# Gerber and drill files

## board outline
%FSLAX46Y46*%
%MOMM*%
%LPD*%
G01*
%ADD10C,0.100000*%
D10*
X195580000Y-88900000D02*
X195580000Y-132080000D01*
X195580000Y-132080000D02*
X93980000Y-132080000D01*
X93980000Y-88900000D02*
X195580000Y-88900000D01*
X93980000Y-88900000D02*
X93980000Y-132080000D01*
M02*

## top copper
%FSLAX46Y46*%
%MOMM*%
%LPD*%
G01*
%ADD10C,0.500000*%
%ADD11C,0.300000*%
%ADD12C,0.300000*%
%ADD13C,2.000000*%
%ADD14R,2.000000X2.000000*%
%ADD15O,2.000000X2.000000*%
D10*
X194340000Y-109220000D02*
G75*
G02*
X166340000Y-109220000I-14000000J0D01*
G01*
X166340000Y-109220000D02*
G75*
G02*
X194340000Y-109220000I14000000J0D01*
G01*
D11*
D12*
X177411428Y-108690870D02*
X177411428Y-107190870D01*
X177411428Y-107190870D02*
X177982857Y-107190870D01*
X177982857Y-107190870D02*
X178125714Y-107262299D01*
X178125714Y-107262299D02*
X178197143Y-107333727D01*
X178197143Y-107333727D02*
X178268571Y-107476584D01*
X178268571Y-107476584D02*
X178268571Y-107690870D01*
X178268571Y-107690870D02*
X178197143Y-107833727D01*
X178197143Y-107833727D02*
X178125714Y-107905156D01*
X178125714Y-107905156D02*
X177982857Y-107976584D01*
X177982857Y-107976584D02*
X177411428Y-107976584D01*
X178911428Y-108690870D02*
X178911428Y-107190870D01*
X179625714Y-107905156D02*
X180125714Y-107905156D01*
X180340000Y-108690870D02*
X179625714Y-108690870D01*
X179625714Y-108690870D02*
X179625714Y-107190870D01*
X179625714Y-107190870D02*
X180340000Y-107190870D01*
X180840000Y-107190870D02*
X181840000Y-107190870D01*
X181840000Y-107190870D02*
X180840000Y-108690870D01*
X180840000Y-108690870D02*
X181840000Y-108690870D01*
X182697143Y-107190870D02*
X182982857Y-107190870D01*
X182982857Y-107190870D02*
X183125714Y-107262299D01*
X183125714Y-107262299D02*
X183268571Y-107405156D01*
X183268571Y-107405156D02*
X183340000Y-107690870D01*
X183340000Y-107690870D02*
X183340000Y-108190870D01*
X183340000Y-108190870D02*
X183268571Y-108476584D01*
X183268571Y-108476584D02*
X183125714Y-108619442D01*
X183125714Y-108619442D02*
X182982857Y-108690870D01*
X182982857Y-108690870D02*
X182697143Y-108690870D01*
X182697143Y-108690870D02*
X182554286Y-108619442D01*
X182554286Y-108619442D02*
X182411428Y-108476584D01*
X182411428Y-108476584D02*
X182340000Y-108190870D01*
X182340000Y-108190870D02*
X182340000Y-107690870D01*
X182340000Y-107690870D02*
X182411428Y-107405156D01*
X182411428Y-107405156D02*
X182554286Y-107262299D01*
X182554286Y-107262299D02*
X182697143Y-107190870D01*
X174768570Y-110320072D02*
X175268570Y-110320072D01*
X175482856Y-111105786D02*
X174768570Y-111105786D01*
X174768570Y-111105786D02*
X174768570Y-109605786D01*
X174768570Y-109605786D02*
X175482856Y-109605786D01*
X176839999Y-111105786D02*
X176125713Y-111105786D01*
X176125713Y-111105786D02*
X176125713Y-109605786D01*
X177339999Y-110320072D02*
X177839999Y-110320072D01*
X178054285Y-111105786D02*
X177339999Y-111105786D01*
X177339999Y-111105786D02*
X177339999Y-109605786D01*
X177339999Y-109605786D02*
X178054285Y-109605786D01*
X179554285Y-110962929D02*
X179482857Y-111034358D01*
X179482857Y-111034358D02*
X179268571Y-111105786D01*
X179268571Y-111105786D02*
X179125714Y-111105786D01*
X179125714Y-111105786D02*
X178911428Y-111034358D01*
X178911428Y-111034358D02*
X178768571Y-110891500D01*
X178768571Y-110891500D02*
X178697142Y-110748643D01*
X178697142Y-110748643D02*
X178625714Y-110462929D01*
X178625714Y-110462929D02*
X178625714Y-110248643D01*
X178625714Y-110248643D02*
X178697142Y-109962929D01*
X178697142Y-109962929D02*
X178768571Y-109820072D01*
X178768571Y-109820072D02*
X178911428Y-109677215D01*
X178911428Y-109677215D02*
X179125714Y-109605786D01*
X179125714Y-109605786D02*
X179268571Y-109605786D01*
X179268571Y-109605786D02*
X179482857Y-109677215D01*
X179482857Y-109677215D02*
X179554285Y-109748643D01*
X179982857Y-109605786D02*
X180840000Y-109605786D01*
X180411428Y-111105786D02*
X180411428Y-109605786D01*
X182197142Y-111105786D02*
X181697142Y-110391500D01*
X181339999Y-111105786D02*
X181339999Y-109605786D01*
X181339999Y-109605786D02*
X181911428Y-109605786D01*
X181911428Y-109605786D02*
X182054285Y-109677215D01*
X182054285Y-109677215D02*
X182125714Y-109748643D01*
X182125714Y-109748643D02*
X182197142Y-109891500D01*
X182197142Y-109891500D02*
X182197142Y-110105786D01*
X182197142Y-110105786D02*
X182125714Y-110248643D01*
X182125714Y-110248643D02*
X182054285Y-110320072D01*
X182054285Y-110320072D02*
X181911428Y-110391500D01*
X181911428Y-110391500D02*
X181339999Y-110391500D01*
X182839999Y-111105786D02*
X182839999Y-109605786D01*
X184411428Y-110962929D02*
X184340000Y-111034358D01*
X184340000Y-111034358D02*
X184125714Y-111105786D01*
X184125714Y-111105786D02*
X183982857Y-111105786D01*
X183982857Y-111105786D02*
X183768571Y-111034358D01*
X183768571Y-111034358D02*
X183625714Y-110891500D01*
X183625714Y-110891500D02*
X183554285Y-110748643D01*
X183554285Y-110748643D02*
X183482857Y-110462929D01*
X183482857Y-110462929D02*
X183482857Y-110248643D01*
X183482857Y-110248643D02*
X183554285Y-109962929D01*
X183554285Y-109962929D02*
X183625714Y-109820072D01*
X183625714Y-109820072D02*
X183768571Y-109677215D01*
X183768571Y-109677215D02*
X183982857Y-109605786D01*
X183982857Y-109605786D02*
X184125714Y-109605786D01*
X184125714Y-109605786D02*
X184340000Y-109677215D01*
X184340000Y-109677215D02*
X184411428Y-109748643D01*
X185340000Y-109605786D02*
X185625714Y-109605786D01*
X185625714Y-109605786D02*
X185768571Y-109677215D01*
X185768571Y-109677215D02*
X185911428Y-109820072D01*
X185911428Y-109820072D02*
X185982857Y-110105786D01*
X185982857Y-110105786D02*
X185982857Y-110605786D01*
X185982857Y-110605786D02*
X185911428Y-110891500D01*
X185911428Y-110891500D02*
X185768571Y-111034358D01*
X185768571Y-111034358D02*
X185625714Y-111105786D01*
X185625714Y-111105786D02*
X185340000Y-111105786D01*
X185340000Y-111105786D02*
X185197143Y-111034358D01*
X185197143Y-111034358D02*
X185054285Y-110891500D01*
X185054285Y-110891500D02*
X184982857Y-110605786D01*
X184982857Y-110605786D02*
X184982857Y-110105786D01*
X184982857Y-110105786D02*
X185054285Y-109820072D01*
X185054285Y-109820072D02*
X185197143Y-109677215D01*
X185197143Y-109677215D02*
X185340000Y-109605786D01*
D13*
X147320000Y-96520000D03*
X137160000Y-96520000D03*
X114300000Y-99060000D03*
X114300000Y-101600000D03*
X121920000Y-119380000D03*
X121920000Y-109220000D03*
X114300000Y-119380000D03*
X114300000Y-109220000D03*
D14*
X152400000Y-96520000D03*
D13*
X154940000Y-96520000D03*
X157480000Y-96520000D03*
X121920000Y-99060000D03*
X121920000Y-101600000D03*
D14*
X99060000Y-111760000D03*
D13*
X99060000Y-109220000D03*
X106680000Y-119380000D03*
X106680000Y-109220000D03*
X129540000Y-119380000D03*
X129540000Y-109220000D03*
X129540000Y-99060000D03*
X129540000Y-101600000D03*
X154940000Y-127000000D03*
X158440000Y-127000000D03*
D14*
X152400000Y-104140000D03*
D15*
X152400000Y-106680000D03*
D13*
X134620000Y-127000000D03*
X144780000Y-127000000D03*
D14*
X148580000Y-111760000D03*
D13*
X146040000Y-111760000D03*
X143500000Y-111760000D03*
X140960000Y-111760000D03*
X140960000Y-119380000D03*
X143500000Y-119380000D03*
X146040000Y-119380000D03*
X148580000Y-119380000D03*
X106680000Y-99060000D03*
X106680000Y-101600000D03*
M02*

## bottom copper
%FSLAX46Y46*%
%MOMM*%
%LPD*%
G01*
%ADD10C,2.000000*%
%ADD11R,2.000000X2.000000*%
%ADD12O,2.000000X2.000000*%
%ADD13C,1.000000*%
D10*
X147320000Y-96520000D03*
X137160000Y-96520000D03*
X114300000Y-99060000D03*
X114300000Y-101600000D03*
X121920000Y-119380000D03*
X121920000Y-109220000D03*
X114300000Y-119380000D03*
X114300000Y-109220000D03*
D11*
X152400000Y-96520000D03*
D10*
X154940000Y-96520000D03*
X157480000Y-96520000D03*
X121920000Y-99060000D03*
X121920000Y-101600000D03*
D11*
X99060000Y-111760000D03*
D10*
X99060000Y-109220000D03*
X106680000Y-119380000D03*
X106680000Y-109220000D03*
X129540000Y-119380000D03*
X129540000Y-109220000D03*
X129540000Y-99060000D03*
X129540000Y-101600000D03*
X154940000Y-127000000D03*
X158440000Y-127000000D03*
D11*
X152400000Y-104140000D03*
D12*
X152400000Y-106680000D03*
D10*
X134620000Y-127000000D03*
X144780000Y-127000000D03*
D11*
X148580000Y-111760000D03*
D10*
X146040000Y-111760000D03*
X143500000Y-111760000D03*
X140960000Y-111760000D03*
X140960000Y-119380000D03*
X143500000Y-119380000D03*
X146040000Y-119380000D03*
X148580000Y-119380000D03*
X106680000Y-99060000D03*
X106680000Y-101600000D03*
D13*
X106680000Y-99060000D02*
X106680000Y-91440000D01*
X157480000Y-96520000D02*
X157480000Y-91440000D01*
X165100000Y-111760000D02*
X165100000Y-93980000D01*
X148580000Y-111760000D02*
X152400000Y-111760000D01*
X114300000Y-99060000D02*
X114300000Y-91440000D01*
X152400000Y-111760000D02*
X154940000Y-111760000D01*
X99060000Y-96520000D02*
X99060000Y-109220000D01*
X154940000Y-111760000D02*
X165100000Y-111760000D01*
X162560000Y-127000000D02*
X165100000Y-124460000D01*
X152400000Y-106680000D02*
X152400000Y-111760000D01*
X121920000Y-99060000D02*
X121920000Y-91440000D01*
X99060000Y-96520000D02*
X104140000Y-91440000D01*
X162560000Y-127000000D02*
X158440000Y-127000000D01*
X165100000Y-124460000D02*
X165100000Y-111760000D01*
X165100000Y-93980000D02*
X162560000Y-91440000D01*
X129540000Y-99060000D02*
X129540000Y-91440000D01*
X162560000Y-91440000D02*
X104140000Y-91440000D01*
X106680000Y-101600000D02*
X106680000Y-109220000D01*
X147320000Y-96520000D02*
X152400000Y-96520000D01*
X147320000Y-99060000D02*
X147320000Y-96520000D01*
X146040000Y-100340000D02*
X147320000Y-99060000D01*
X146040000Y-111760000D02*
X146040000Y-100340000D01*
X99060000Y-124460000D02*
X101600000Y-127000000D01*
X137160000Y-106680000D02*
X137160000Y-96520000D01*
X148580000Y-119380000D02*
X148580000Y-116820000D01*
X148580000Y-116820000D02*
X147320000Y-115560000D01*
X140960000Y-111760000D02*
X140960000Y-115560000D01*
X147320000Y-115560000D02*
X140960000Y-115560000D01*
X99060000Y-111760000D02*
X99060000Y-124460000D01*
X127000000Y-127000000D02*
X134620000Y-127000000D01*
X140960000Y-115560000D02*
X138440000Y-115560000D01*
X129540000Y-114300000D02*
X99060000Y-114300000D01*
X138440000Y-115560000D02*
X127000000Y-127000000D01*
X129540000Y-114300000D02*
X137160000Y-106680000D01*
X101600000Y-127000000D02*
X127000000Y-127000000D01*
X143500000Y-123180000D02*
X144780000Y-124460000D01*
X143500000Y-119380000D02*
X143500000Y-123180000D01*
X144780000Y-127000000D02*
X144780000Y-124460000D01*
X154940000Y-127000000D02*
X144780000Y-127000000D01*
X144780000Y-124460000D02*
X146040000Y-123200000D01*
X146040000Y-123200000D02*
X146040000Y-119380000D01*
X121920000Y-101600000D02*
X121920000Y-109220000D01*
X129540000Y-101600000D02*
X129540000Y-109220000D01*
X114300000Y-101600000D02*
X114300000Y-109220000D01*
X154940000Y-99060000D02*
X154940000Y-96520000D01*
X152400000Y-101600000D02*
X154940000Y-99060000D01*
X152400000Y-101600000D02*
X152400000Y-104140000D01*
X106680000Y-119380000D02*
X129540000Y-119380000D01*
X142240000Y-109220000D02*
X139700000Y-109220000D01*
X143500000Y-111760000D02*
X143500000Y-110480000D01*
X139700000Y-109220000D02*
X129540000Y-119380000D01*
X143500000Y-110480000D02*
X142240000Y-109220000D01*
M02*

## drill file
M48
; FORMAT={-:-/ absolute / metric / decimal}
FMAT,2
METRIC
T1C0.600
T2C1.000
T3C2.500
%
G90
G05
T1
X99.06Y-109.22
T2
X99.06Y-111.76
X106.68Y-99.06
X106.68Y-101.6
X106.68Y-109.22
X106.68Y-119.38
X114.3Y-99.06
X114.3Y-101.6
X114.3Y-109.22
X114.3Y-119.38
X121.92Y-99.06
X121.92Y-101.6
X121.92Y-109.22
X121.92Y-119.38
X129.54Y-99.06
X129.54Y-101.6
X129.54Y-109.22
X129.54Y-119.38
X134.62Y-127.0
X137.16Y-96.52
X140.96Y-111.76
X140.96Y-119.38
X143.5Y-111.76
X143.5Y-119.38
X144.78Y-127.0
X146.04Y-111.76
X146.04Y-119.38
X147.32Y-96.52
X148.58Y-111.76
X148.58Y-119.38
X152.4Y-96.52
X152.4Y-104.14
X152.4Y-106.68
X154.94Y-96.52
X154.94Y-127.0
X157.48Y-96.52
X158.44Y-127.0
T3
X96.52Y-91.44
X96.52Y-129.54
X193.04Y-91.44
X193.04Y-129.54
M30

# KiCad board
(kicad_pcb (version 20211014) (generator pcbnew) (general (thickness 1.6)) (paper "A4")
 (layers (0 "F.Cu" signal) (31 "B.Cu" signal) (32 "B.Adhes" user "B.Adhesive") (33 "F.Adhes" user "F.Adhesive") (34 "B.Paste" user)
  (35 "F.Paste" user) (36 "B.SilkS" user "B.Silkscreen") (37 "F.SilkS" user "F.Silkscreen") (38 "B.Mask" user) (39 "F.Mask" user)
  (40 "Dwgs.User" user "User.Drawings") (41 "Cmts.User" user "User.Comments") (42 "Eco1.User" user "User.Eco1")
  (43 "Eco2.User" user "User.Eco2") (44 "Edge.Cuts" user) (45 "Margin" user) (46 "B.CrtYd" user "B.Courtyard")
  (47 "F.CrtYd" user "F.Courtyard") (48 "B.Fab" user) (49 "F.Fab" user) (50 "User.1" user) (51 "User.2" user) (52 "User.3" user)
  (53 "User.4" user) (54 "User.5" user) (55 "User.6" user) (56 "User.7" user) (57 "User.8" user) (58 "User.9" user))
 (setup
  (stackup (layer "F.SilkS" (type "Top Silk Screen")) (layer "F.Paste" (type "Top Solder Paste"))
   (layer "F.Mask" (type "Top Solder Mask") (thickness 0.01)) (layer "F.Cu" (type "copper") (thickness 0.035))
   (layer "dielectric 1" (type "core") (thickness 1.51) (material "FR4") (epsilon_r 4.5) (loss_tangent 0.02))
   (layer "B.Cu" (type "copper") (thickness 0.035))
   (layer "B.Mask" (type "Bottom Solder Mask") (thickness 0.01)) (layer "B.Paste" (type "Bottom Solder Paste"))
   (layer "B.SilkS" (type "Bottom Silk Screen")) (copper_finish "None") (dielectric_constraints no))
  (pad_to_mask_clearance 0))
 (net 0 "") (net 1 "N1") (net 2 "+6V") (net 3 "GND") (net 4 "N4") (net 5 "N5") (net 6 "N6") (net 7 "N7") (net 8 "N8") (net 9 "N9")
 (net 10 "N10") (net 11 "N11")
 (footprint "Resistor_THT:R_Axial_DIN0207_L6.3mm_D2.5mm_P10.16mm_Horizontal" (layer "F.Cu") (at 147.32 96.52 180)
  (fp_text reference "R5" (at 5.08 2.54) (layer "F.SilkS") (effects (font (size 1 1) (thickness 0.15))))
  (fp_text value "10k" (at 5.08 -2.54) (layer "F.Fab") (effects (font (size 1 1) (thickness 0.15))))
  (pad "1" thru_hole circle (at 0 0 180) (size 2 2) (drill 1) (layers *.Cu *.Mask) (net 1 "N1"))
  (pad "2" thru_hole circle (at 10.16 0 180) (size 2 2) (drill 1) (layers *.Cu *.Mask) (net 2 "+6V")))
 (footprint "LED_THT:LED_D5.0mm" (layer "F.Cu") (at 114.3 99.06 -90)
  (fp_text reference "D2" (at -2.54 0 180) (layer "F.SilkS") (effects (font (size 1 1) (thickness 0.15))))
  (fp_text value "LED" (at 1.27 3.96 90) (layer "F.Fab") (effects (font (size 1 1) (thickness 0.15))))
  (pad "1" thru_hole circle (at 0 0 270) (size 2 2) (drill 1) (layers *.Cu *.Mask) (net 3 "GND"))
  (pad "2" thru_hole circle (at 2.54 0 270) (size 2 2) (drill 1) (layers *.Cu *.Mask) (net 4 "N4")))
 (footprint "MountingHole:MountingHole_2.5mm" (layer "F.Cu") (at 96.52 91.44)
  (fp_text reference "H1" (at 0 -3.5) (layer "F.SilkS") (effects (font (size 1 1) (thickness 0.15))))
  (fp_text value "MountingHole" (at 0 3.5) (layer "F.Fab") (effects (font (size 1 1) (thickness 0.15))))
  (pad "" np_thru_hole circle (at 0 0) (size 2.5 2.5) (drill 2.5) (layers *.Cu *.Mask)))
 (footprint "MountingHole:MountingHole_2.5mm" (layer "F.Cu") (at 96.52 129.54 180)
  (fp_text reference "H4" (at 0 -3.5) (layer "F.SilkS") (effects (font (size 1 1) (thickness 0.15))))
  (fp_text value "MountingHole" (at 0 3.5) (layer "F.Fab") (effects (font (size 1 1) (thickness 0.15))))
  (pad "" np_thru_hole circle (at 0 0 180) (size 2.5 2.5) (drill 2.5) (layers *.Cu *.Mask)))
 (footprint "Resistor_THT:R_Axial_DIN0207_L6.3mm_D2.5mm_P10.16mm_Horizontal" (layer "F.Cu") (at 121.92 119.38 90)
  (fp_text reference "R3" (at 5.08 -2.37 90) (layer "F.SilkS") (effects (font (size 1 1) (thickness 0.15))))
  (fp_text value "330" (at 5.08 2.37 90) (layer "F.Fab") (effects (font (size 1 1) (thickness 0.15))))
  (pad "1" thru_hole circle (at 0 0 90) (size 2 2) (drill 1) (layers *.Cu *.Mask) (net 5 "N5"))
  (pad "2" thru_hole circle (at 10.16 0 90) (size 2 2) (drill 1) (layers *.Cu *.Mask) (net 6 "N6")))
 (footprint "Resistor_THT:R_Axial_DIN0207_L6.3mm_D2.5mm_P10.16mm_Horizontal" (layer "F.Cu") (at 114.3 119.38 90)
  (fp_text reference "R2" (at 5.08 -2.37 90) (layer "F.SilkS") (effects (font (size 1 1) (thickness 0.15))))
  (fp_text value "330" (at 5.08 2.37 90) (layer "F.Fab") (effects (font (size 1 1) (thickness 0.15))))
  (pad "1" thru_hole circle (at 0 0 90) (size 2 2) (drill 1) (layers *.Cu *.Mask) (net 5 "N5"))
  (pad "2" thru_hole circle (at 10.16 0 90) (size 2 2) (drill 1) (layers *.Cu *.Mask) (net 4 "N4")))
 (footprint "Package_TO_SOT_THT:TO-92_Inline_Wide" (layer "F.Cu") (at 152.4 96.52)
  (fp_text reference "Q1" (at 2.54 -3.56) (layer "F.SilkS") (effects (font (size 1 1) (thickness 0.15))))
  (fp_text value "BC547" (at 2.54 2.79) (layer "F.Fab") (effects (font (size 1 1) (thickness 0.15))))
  (pad "1" thru_hole rect (at 0 0) (size 2 2) (drill 1) (layers *.Cu *.Mask) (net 1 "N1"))
  (pad "2" thru_hole circle (at 2.54 0) (size 2 2) (drill 1) (layers *.Cu *.Mask) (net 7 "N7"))
  (pad "3" thru_hole circle (at 5.08 0) (size 2 2) (drill 1) (layers *.Cu *.Mask) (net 3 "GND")))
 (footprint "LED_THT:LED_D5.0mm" (layer "F.Cu") (at 121.92 99.06 -90)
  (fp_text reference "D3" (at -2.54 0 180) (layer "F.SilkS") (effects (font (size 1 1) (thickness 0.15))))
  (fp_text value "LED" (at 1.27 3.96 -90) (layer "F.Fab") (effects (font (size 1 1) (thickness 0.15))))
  (pad "1" thru_hole circle (at 0 0 270) (size 2 2) (drill 1) (layers *.Cu *.Mask) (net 3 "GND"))
  (pad "2" thru_hole circle (at 2.54 0 270) (size 2 2) (drill 1) (layers *.Cu *.Mask) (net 6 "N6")))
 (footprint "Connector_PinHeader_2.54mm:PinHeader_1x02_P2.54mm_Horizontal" (layer "F.Cu") (at 99.06 111.76 180)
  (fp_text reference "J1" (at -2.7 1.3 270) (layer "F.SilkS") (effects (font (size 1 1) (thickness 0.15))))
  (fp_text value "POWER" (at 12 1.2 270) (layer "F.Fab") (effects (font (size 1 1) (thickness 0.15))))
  (pad "1" thru_hole rect (at 0 0 180) (size 2 2) (drill 1) (layers *.Cu *.Mask) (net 2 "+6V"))
  (pad "2" thru_hole circle (at 0 2.54 180) (size 2 2) (drill 0.6) (layers *.Cu *.Mask) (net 3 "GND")))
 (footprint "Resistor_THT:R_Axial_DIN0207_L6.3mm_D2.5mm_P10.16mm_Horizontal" (layer "F.Cu") (at 106.68 119.38 90)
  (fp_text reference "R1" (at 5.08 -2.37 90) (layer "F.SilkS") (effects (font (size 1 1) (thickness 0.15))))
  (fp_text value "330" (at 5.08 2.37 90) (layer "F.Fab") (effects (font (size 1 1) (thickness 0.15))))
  (pad "1" thru_hole circle (at 0 0 90) (size 2 2) (drill 1) (layers *.Cu *.Mask) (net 5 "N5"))
  (pad "2" thru_hole circle (at 10.16 0 90) (size 2 2) (drill 1) (layers *.Cu *.Mask) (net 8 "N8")))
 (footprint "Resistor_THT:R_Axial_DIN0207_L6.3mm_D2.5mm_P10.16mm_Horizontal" (layer "F.Cu") (at 129.54 119.38 90)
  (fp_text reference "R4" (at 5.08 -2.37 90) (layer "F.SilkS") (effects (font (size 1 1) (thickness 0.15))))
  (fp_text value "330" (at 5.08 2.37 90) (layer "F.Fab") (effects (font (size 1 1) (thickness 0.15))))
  (pad "1" thru_hole circle (at 0 0 90) (size 2 2) (drill 1) (layers *.Cu *.Mask) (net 5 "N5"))
  (pad "2" thru_hole circle (at 10.16 0 90) (size 2 2) (drill 1) (layers *.Cu *.Mask "Dwgs.User") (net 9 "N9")))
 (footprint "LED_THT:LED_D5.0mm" (layer "F.Cu") (at 129.54 99.06 -90)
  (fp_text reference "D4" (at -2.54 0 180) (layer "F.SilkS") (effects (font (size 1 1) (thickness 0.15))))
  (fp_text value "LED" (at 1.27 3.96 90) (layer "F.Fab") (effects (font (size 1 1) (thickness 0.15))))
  (pad "1" thru_hole circle (at 0 0 270) (size 2 2) (drill 1) (layers *.Cu *.Mask) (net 3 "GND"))
  (pad "2" thru_hole circle (at 2.54 0 270) (size 2 2) (drill 1) (layers *.Cu "B.Mask") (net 9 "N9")))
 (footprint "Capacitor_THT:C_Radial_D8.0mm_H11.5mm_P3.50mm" (layer "F.Cu") (at 154.94 127)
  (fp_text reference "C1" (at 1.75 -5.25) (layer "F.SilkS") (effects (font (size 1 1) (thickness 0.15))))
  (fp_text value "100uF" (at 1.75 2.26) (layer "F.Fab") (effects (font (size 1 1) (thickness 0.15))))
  (pad "1" thru_hole circle (at 0 0) (size 2 2) (drill 1) (layers *.Cu *.Mask) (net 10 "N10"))
  (pad "2" thru_hole circle (at 3.5 0) (size 2 2) (drill 1) (layers *.Cu *.Mask) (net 3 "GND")))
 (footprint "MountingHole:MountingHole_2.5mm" (layer "F.Cu") (at 193.04 91.44)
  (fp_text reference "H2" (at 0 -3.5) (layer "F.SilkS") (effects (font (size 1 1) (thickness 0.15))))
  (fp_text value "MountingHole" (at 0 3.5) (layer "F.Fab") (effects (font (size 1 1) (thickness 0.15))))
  (pad "" np_thru_hole circle (at 0 0) (size 2.5 2.5) (drill 2.5) (layers *.Cu *.Mask)))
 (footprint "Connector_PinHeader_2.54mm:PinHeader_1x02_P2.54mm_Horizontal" (layer "F.Cu") (at 152.4 104.14)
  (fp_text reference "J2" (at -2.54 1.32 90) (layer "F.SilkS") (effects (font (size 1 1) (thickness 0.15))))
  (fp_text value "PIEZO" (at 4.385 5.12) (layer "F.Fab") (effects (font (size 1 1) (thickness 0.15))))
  (pad "1" thru_hole rect (at 0 0) (size 2 2) (drill 1) (layers *.Cu *.Mask) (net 7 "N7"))
  (pad "2" thru_hole oval (at 0 2.54) (size 2 2) (drill 1) (layers *.Cu *.Mask) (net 3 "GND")))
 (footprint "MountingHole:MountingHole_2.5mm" (layer "F.Cu") (at 193.04 129.54 180)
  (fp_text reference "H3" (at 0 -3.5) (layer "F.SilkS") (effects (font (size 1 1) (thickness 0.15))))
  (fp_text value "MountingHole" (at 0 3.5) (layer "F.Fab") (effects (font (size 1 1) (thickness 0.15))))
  (pad "" np_thru_hole circle (at 0 0 180) (size 2.5 2.5) (drill 2.5) (layers *.Cu *.Mask)))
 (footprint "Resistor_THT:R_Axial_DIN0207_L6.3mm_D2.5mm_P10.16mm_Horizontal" (layer "F.Cu") (at 134.62 127)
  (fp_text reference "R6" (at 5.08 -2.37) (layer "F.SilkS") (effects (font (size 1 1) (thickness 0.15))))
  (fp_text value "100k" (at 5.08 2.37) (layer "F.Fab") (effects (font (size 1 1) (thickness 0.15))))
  (pad "1" thru_hole circle (at 0 0) (size 2 2) (drill 1) (layers *.Cu *.Mask) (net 2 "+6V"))
  (pad "2" thru_hole circle (at 10.16 0) (size 2 2) (drill 1) (layers *.Cu *.Mask) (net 10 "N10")))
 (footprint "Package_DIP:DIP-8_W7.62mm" (layer "F.Cu") (at 148.58 111.76 -90)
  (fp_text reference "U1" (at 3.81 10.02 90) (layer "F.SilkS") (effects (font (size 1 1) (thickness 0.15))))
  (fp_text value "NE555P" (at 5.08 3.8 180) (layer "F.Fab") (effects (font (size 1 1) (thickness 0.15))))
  (pad "1" thru_hole rect (at 0 0 270) (size 2 2) (drill 1) (layers *.Cu *.Mask) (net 3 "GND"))
  (pad "2" thru_hole circle (at 0 2.54 270) (size 2 2) (drill 1) (layers *.Cu *.Mask) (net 1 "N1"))
  (pad "3" thru_hole circle (at 0 5.08 270) (size 2 2) (drill 1) (layers *.Cu *.Mask) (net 5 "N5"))
  (pad "4" thru_hole circle (at 0 7.62 270) (size 2 2) (drill 1) (layers *.Cu *.Mask) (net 2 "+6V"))
  (pad "5" thru_hole circle (at 7.62 7.62 270) (size 2 2) (drill 1) (layers *.Cu *.Mask) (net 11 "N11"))
  (pad "6" thru_hole circle (at 7.62 5.08 270) (size 2 2) (drill 1) (layers *.Cu *.Mask) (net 10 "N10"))
  (pad "7" thru_hole circle (at 7.62 2.54 270) (size 2 2) (drill 1) (layers *.Cu *.Mask) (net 10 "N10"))
  (pad "8" thru_hole circle (at 7.62 0 270) (size 2 2) (drill 1) (layers *.Cu *.Mask) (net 2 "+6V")))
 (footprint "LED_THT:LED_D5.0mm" (layer "F.Cu") (at 106.68 99.06 -90)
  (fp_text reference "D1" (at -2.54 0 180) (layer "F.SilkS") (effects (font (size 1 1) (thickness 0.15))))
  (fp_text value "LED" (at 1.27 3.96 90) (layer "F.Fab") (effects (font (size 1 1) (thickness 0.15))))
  (pad "1" thru_hole circle (at 0 0 270) (size 2 2) (drill 1) (layers *.Cu *.Mask) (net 3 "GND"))
  (pad "2" thru_hole circle (at 2.54 0 270) (size 2 2) (drill 1) (layers *.Cu *.Mask) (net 8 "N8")))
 (gr_circle (center 180.34 109.22) (end 194.34 109.22) (layer "F.Cu") (width 0.5) (fill none))
 (gr_line (start 195.58 88.9) (end 195.58 132.08) (layer "Edge.Cuts") (width 0.1))
 (gr_line (start 195.58 132.08) (end 93.98 132.08) (layer "Edge.Cuts") (width 0.1))
 (gr_line (start 93.98 88.9) (end 195.58 88.9) (layer "Edge.Cuts") (width 0.1))
 (gr_line (start 93.98 88.9) (end 93.98 132.08) (layer "Edge.Cuts") (width 0.1))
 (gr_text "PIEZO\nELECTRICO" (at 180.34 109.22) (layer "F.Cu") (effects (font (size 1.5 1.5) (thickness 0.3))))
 (segment (start 106.68 99.06) (end 106.68 91.44) (width 1) (layer "B.Cu") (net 3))
 (segment (start 157.48 96.52) (end 157.48 91.44) (width 1) (layer "B.Cu") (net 3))
 (segment (start 165.1 111.76) (end 165.1 93.98) (width 1) (layer "B.Cu") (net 3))
 (segment (start 148.58 111.76) (end 152.4 111.76) (width 1) (layer "B.Cu") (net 3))
 (segment (start 114.3 99.06) (end 114.3 91.44) (width 1) (layer "B.Cu") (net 3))
 (segment (start 152.4 111.76) (end 154.94 111.76) (width 1) (layer "B.Cu") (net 3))
 (segment (start 99.06 96.52) (end 99.06 109.22) (width 1) (layer "B.Cu") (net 3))
 (segment (start 154.94 111.76) (end 165.1 111.76) (width 1) (layer "B.Cu") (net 3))
 (segment (start 162.56 127) (end 165.1 124.46) (width 1) (layer "B.Cu") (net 3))
 (segment (start 152.4 106.68) (end 152.4 111.76) (width 1) (layer "B.Cu") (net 3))
 (segment (start 121.92 99.06) (end 121.92 91.44) (width 1) (layer "B.Cu") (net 3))
 (segment (start 99.06 96.52) (end 104.14 91.44) (width 1) (layer "B.Cu") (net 3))
 (segment (start 162.56 127) (end 158.44 127) (width 1) (layer "B.Cu") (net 3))
 (segment (start 165.1 124.46) (end 165.1 111.76) (width 1) (layer "B.Cu") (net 3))
 (segment (start 165.1 93.98) (end 162.56 91.44) (width 1) (layer "B.Cu") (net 3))
 (segment (start 129.54 99.06) (end 129.54 91.44) (width 1) (layer "B.Cu") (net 3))
 (segment (start 162.56 91.44) (end 104.14 91.44) (width 1) (layer "B.Cu") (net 3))
 (segment (start 106.68 101.6) (end 106.68 109.22) (width 1) (layer "B.Cu") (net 8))
 (segment (start 147.32 96.52) (end 152.4 96.52) (width 1) (layer "B.Cu") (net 1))
 (segment (start 147.32 99.06) (end 147.32 96.52) (width 1) (layer "B.Cu") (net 1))
 (segment (start 146.04 100.34) (end 147.32 99.06) (width 1) (layer "B.Cu") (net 1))
 (segment (start 146.04 111.76) (end 146.04 100.34) (width 1) (layer "B.Cu") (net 1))
 (segment (start 99.06 124.46) (end 101.6 127) (width 1) (layer "B.Cu") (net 2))
 (segment (start 137.16 106.68) (end 137.16 96.52) (width 1) (layer "B.Cu") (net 2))
 (segment (start 148.58 119.38) (end 148.58 116.82) (width 1) (layer "B.Cu") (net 2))
 (segment (start 148.58 116.82) (end 147.32 115.56) (width 1) (layer "B.Cu") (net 2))
 (segment (start 140.96 111.76) (end 140.96 115.56) (width 1) (layer "B.Cu") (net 2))
 (segment (start 147.32 115.56) (end 140.96 115.56) (width 1) (layer "B.Cu") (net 2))
 (segment (start 99.06 111.76) (end 99.06 124.46) (width 1) (layer "B.Cu") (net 2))
 (segment (start 127 127) (end 134.62 127) (width 1) (layer "B.Cu") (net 2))
 (segment (start 140.96 115.56) (end 138.44 115.56) (width 1) (layer "B.Cu") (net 2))
 (segment (start 129.54 114.3) (end 99.06 114.3) (width 1) (layer "B.Cu") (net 2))
 (segment (start 138.44 115.56) (end 127 127) (width 1) (layer "B.Cu") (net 2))
 (segment (start 129.54 114.3) (end 137.16 106.68) (width 1) (layer "B.Cu") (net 2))
 (segment (start 101.6 127) (end 127 127) (width 1) (layer "B.Cu") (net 2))
 (segment (start 143.5 123.18) (end 144.78 124.46) (width 1) (layer "B.Cu") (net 10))
 (segment (start 143.5 119.38) (end 143.5 123.18) (width 1) (layer "B.Cu") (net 10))
 (segment (start 144.78 127) (end 144.78 124.46) (width 1) (layer "B.Cu") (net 10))
 (segment (start 154.94 127) (end 144.78 127) (width 1) (layer "B.Cu") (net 10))
 (segment (start 144.78 124.46) (end 146.04 123.2) (width 1) (layer "B.Cu") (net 10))
 (segment (start 146.04 123.2) (end 146.04 119.38) (width 1) (layer "B.Cu") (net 10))
 (segment (start 121.92 101.6) (end 121.92 109.22) (width 1) (layer "B.Cu") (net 6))
 (segment (start 129.54 101.6) (end 129.54 109.22) (width 1) (layer "B.Cu") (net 9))
 (segment (start 114.3 101.6) (end 114.3 109.22) (width 1) (layer "B.Cu") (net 4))
 (segment (start 154.94 99.06) (end 154.94 96.52) (width 1) (layer "B.Cu") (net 7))
 (segment (start 152.4 101.6) (end 154.94 99.06) (width 1) (layer "B.Cu") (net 7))
 (segment (start 152.4 101.6) (end 152.4 104.14) (width 1) (layer "B.Cu") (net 7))
 (segment (start 106.68 119.38) (end 129.54 119.38) (width 1) (layer "B.Cu") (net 5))
 (segment (start 142.24 109.22) (end 139.7 109.22) (width 1) (layer "B.Cu") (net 5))
 (segment (start 143.5 111.76) (end 143.5 110.48) (width 1) (layer "B.Cu") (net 5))
 (segment (start 139.7 109.22) (end 129.54 119.38) (width 1) (layer "B.Cu") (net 5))
 (segment (start 143.5 110.48) (end 142.24 109.22) (width 1) (layer "B.Cu") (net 5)))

